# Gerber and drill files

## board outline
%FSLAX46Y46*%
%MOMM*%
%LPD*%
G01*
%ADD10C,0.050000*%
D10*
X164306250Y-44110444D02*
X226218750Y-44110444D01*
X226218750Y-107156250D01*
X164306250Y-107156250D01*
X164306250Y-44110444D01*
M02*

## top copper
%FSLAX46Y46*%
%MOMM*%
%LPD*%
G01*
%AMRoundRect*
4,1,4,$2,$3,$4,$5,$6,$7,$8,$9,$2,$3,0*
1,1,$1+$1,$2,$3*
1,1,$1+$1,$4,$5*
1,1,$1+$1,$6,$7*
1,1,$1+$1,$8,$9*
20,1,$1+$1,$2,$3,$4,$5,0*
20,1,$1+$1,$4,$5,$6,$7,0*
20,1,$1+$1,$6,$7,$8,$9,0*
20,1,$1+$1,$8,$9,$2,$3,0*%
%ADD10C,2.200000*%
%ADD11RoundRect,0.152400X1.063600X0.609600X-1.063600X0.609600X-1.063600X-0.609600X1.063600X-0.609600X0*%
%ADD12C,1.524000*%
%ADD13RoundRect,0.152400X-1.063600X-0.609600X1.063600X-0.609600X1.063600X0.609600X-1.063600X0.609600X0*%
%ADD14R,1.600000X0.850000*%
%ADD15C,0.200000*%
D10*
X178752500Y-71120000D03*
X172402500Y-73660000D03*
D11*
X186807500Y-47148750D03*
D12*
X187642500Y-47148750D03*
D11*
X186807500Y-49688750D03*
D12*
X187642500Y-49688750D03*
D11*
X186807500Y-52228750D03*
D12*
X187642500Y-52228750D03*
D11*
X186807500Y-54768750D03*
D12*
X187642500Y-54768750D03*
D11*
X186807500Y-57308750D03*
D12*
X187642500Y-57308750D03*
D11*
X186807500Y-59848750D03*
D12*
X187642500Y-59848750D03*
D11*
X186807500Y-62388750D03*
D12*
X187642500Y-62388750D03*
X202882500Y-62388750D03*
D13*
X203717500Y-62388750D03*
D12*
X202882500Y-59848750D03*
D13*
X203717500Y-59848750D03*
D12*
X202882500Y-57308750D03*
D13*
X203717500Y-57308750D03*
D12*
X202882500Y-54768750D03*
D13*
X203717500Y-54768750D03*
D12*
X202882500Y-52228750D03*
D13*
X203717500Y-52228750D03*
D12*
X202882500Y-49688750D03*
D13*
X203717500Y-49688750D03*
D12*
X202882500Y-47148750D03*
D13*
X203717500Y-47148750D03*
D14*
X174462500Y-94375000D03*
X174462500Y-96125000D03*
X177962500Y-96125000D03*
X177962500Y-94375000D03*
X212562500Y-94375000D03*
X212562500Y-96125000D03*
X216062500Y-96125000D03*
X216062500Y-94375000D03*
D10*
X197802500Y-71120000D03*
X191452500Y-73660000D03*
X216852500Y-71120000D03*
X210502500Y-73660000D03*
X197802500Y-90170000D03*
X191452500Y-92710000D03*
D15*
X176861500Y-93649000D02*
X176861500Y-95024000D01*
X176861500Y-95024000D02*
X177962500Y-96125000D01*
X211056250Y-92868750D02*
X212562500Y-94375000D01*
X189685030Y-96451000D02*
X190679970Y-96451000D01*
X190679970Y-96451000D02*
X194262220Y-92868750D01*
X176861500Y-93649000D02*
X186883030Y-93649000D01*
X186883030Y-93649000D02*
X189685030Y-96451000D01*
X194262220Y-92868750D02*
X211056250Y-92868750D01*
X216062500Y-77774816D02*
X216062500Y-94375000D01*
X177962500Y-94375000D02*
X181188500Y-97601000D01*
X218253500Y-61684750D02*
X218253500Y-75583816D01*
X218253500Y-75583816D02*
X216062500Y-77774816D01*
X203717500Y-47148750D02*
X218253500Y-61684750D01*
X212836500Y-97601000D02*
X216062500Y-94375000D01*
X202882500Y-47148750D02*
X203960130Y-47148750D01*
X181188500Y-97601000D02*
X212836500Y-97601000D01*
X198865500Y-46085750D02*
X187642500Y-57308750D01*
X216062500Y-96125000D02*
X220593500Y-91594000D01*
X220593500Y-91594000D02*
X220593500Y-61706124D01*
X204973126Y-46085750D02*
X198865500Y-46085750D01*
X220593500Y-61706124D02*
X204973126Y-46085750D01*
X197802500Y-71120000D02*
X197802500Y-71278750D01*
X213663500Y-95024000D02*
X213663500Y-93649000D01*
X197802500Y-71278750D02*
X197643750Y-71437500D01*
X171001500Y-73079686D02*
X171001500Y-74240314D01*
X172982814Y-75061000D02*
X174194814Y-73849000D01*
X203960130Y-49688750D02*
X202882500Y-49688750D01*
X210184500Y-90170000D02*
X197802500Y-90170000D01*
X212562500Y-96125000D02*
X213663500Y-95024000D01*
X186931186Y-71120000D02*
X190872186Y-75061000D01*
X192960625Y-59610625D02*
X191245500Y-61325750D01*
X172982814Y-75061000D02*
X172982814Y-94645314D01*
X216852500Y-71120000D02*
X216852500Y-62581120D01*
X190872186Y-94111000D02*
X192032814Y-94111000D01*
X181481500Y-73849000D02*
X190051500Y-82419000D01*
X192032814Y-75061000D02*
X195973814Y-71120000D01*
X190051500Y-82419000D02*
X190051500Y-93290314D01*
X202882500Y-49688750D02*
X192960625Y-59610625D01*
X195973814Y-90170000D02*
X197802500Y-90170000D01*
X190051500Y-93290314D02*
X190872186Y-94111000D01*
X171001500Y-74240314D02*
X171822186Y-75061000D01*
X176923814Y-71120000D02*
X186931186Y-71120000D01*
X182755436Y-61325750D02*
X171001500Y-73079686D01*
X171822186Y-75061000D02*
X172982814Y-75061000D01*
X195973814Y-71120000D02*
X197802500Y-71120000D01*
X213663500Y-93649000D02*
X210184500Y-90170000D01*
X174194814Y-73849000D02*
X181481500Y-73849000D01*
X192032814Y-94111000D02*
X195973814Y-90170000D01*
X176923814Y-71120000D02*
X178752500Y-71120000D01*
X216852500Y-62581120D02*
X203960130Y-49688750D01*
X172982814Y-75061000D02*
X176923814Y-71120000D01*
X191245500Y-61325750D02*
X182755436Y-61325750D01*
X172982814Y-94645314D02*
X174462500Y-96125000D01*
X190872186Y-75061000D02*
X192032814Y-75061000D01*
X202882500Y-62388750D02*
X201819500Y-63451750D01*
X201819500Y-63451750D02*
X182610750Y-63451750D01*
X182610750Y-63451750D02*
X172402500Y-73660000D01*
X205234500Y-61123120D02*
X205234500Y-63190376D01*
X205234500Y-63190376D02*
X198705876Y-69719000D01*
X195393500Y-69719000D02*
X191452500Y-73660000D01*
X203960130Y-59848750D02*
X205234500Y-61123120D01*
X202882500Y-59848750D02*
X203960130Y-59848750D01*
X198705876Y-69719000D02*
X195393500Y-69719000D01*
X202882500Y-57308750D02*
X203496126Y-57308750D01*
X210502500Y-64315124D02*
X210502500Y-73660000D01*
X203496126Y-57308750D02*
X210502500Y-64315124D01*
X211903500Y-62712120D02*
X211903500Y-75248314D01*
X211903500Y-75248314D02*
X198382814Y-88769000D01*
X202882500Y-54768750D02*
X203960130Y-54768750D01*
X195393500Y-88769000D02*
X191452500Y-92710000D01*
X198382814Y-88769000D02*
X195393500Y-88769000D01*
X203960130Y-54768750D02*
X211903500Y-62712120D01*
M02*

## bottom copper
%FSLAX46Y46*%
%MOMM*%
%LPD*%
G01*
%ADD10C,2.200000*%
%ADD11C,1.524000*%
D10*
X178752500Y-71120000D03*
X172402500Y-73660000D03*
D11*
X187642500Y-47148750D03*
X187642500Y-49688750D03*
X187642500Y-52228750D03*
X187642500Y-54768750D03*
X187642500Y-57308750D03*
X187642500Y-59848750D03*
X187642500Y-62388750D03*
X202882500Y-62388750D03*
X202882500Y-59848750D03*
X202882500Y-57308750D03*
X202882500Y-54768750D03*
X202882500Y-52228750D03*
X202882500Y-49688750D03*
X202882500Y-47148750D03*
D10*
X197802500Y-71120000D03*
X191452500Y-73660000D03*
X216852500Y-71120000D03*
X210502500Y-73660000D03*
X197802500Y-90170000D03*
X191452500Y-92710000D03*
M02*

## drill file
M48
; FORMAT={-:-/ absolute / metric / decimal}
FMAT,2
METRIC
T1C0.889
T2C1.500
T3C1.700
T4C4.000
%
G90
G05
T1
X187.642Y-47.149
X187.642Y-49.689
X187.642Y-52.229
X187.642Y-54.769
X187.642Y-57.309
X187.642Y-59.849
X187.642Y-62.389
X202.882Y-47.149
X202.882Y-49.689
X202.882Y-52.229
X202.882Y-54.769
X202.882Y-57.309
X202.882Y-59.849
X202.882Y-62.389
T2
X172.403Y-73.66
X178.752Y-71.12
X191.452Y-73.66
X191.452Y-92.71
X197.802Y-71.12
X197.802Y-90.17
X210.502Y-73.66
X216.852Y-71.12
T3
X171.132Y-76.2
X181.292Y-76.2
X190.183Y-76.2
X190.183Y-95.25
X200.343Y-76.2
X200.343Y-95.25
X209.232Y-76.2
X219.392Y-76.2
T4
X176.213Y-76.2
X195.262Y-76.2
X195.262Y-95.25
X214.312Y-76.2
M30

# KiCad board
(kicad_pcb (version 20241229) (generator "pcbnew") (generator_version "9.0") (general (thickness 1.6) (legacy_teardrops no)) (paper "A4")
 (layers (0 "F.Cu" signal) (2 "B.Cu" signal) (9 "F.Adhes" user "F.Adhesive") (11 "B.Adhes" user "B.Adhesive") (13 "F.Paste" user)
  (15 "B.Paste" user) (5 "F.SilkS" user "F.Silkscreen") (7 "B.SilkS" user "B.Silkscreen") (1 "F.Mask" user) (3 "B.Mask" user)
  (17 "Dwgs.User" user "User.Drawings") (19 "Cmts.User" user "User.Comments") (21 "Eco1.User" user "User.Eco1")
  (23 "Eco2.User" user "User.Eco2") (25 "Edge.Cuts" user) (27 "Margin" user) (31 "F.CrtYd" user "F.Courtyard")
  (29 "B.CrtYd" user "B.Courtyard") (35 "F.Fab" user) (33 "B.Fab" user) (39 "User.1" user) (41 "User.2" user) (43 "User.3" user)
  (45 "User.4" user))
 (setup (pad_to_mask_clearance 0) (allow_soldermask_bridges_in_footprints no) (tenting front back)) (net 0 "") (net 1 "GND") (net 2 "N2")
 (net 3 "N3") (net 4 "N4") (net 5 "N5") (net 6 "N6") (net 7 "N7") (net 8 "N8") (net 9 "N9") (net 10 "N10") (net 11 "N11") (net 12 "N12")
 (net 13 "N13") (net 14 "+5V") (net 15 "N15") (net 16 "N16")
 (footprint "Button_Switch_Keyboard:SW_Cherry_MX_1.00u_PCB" (layer "F.Cu") (at 178.7525 71.12)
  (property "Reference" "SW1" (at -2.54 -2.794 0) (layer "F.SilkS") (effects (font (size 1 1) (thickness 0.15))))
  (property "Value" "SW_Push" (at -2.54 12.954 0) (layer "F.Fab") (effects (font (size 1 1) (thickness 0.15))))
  (pad "" np_thru_hole circle (at -7.62 5.08) (size 1.7 1.7) (drill 1.7) (layers "*.Cu" "*.Mask"))
  (pad "" np_thru_hole circle (at -2.54 5.08) (size 4 4) (drill 4) (layers "*.Cu" "*.Mask"))
  (pad "" np_thru_hole circle (at 2.54 5.08) (size 1.7 1.7) (drill 1.7) (layers "*.Cu" "*.Mask"))
  (pad "1" thru_hole circle (at 0 0) (size 2.2 2.2) (drill 1.5) (layers "*.Cu" "*.Mask") (remove_unused_layers no) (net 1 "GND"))
  (pad "2" thru_hole circle (at -6.35 2.54) (size 2.2 2.2) (drill 1.5) (layers "*.Cu" "*.Mask") (remove_unused_layers no) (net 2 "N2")))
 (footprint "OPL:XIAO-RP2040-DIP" (layer "F.Cu") (at 195.2625 54.76875)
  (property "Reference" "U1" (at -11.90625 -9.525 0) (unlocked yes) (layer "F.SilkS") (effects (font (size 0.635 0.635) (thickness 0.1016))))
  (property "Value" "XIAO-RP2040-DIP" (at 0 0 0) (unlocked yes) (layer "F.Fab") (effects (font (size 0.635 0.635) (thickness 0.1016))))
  (pad "1" smd roundrect (at -8.455 -7.62 180) (size 2.432 1.524) (layers "F.Cu" "F.Mask") (roundrect_rratio 0.1) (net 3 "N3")
   (thermal_bridge_angle 45))
  (pad "1" thru_hole circle (at -7.62 -7.62 180) (size 1.524 1.524) (drill 0.889) (layers "*.Cu" "*.Mask") (remove_unused_layers no)
   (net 3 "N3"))
  (pad "2" smd roundrect (at -8.455 -5.08 180) (size 2.432 1.524) (layers "F.Cu" "F.Mask") (roundrect_rratio 0.1) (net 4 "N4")
   (thermal_bridge_angle 45))
  (pad "2" thru_hole circle (at -7.62 -5.08 180) (size 1.524 1.524) (drill 0.889) (layers "*.Cu" "*.Mask") (remove_unused_layers no)
   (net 4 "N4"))
  (pad "3" smd roundrect (at -8.455 -2.54 180) (size 2.432 1.524) (layers "F.Cu" "F.Mask") (roundrect_rratio 0.1) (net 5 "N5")
   (thermal_bridge_angle 45))
  (pad "3" thru_hole circle (at -7.62 -2.54 180) (size 1.524 1.524) (drill 0.889) (layers "*.Cu" "*.Mask") (remove_unused_layers no)
   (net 5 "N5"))
  (pad "4" smd roundrect (at -8.455 0 180) (size 2.432 1.524) (layers "F.Cu" "F.Mask") (roundrect_rratio 0.1) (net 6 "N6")
   (thermal_bridge_angle 45))
  (pad "4" thru_hole circle (at -7.62 0 180) (size 1.524 1.524) (drill 0.889) (layers "*.Cu" "*.Mask") (remove_unused_layers no)
   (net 6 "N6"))
  (pad "5" smd roundrect (at -8.455 2.54 180) (size 2.432 1.524) (layers "F.Cu" "F.Mask") (roundrect_rratio 0.1) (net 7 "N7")
   (thermal_bridge_angle 45))
  (pad "5" thru_hole circle (at -7.62 2.54 180) (size 1.524 1.524) (drill 0.889) (layers "*.Cu" "*.Mask") (remove_unused_layers no)
   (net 7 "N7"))
  (pad "6" smd roundrect (at -8.455 5.08 180) (size 2.432 1.524) (layers "F.Cu" "F.Mask") (roundrect_rratio 0.1) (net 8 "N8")
   (thermal_bridge_angle 45))
  (pad "6" thru_hole circle (at -7.62 5.08 180) (size 1.524 1.524) (drill 0.889) (layers "*.Cu" "*.Mask") (remove_unused_layers no)
   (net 8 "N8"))
  (pad "7" smd roundrect (at -8.455 7.62 180) (size 2.432 1.524) (layers "F.Cu" "F.Mask") (roundrect_rratio 0.1) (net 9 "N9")
   (thermal_bridge_angle 45))
  (pad "7" thru_hole circle (at -7.62 7.62 180) (size 1.524 1.524) (drill 0.889) (layers "*.Cu" "*.Mask") (remove_unused_layers no)
   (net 9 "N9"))
  (pad "8" thru_hole circle (at 7.62 7.62) (size 1.524 1.524) (drill 0.889) (layers "*.Cu" "*.Mask") (remove_unused_layers no) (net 2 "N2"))
  (pad "8" smd roundrect (at 8.455 7.62) (size 2.432 1.524) (layers "F.Cu" "F.Mask") (roundrect_rratio 0.1) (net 2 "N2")
   (thermal_bridge_angle 45))
  (pad "9" thru_hole circle (at 7.62 5.08) (size 1.524 1.524) (drill 0.889) (layers "*.Cu" "*.Mask") (remove_unused_layers no)
   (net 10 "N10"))
  (pad "9" smd roundrect (at 8.455 5.08) (size 2.432 1.524) (layers "F.Cu" "F.Mask") (roundrect_rratio 0.1) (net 10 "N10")
   (thermal_bridge_angle 45))
  (pad "10" thru_hole circle (at 7.62 2.54) (size 1.524 1.524) (drill 0.889) (layers "*.Cu" "*.Mask") (remove_unused_layers no)
   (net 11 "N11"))
  (pad "10" smd roundrect (at 8.455 2.54) (size 2.432 1.524) (layers "F.Cu" "F.Mask") (roundrect_rratio 0.1) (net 11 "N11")
   (thermal_bridge_angle 45))
  (pad "11" thru_hole circle (at 7.62 0) (size 1.524 1.524) (drill 0.889) (layers "*.Cu" "*.Mask") (remove_unused_layers no) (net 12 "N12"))
  (pad "11" smd roundrect (at 8.455 0) (size 2.432 1.524) (layers "F.Cu" "F.Mask") (roundrect_rratio 0.1) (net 12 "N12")
   (thermal_bridge_angle 45))
  (pad "12" thru_hole circle (at 7.62 -2.54) (size 1.524 1.524) (drill 0.889) (layers "*.Cu" "*.Mask") (remove_unused_layers no)
   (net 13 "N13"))
  (pad "12" smd roundrect (at 8.455 -2.54) (size 2.432 1.524) (layers "F.Cu" "F.Mask") (roundrect_rratio 0.1) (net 13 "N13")
   (thermal_bridge_angle 45))
  (pad "13" thru_hole circle (at 7.62 -5.08) (size 1.524 1.524) (drill 0.889) (layers "*.Cu" "*.Mask") (remove_unused_layers no)
   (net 1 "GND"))
  (pad "13" smd roundrect (at 8.455 -5.08) (size 2.432 1.524) (layers "F.Cu" "F.Mask") (roundrect_rratio 0.1) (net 1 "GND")
   (thermal_bridge_angle 45))
  (pad "14" thru_hole circle (at 7.62 -7.62) (size 1.524 1.524) (drill 0.889) (layers "*.Cu" "*.Mask") (remove_unused_layers no)
   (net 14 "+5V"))
  (pad "14" smd roundrect (at 8.455 -7.62) (size 2.432 1.524) (layers "F.Cu" "F.Mask") (roundrect_rratio 0.1) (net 14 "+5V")
   (thermal_bridge_angle 45)))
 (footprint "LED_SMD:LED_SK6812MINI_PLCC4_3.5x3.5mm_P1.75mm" (layer "F.Cu") (at 176.2125 95.25)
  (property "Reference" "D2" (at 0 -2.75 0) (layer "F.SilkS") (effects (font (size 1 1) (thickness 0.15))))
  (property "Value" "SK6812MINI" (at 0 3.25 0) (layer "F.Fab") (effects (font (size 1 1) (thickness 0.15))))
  (pad "1" smd rect (at -1.75 -0.875) (size 1.6 0.85) (layers "F.Cu" "F.Mask" "F.Paste") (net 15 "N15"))
  (pad "2" smd rect (at -1.75 0.875) (size 1.6 0.85) (layers "F.Cu" "F.Mask" "F.Paste") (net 1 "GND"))
  (pad "3" smd rect (at 1.75 0.875) (size 1.6 0.85) (layers "F.Cu" "F.Mask" "F.Paste") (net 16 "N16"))
  (pad "4" smd rect (at 1.75 -0.875) (size 1.6 0.85) (layers "F.Cu" "F.Mask" "F.Paste") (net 14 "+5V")))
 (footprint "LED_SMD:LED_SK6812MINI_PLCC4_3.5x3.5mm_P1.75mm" (layer "F.Cu") (at 214.3125 95.25)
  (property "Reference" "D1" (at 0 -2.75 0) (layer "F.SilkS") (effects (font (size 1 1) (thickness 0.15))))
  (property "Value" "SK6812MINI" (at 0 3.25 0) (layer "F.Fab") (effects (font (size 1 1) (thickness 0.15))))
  (pad "1" smd rect (at -1.75 -0.875) (size 1.6 0.85) (layers "F.Cu" "F.Mask" "F.Paste") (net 16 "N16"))
  (pad "2" smd rect (at -1.75 0.875) (size 1.6 0.85) (layers "F.Cu" "F.Mask" "F.Paste") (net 1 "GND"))
  (pad "3" smd rect (at 1.75 0.875) (size 1.6 0.85) (layers "F.Cu" "F.Mask" "F.Paste") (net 7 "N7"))
  (pad "4" smd rect (at 1.75 -0.875) (size 1.6 0.85) (layers "F.Cu" "F.Mask" "F.Paste") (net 14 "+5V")))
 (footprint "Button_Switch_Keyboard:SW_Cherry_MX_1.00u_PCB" (layer "F.Cu") (at 197.8025 71.12)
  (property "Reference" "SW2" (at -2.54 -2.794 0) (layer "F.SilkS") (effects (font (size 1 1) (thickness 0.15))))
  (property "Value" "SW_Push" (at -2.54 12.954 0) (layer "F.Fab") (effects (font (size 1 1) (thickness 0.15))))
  (pad "" np_thru_hole circle (at -7.62 5.08) (size 1.7 1.7) (drill 1.7) (layers "*.Cu" "*.Mask"))
  (pad "" np_thru_hole circle (at -2.54 5.08) (size 4 4) (drill 4) (layers "*.Cu" "*.Mask"))
  (pad "" np_thru_hole circle (at 2.54 5.08) (size 1.7 1.7) (drill 1.7) (layers "*.Cu" "*.Mask"))
  (pad "1" thru_hole circle (at 0 0) (size 2.2 2.2) (drill 1.5) (layers "*.Cu" "*.Mask") (remove_unused_layers no) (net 1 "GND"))
  (pad "2" thru_hole circle (at -6.35 2.54) (size 2.2 2.2) (drill 1.5) (layers "*.Cu" "*.Mask") (remove_unused_layers no) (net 10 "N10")))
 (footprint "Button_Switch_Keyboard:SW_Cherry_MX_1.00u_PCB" (layer "F.Cu") (at 216.8525 71.12)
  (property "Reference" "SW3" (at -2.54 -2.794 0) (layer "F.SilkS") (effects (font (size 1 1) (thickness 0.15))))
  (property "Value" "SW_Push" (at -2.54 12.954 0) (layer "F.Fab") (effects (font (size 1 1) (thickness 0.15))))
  (pad "" np_thru_hole circle (at -7.62 5.08) (size 1.7 1.7) (drill 1.7) (layers "*.Cu" "*.Mask"))
  (pad "" np_thru_hole circle (at -2.54 5.08) (size 4 4) (drill 4) (layers "*.Cu" "*.Mask"))
  (pad "" np_thru_hole circle (at 2.54 5.08) (size 1.7 1.7) (drill 1.7) (layers "*.Cu" "*.Mask"))
  (pad "1" thru_hole circle (at 0 0) (size 2.2 2.2) (drill 1.5) (layers "*.Cu" "*.Mask") (remove_unused_layers no) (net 1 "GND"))
  (pad "2" thru_hole circle (at -6.35 2.54) (size 2.2 2.2) (drill 1.5) (layers "*.Cu" "*.Mask") (remove_unused_layers no) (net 11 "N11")))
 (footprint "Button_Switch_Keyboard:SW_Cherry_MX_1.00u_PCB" (layer "F.Cu") (at 197.8025 90.17)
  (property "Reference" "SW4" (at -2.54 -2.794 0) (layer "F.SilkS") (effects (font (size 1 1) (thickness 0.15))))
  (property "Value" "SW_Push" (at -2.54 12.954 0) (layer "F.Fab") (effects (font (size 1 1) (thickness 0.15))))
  (pad "" np_thru_hole circle (at -7.62 5.08) (size 1.7 1.7) (drill 1.7) (layers "*.Cu" "*.Mask"))
  (pad "" np_thru_hole circle (at -2.54 5.08) (size 4 4) (drill 4) (layers "*.Cu" "*.Mask"))
  (pad "" np_thru_hole circle (at 2.54 5.08) (size 1.7 1.7) (drill 1.7) (layers "*.Cu" "*.Mask"))
  (pad "1" thru_hole circle (at 0 0) (size 2.2 2.2) (drill 1.5) (layers "*.Cu" "*.Mask") (remove_unused_layers no) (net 1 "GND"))
  (pad "2" thru_hole circle (at -6.35 2.54) (size 2.2 2.2) (drill 1.5) (layers "*.Cu" "*.Mask") (remove_unused_layers no) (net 12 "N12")))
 (gr_rect (start 164.30625 44.110444) (end 226.21875 107.15625) (stroke (width 0.05) (type default)) (fill no) (layer "Edge.Cuts"))
 (segment (start 176.8615 93.649) (end 176.8615 95.024) (width 0.2) (layer "F.Cu") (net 16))
 (segment (start 176.8615 95.024) (end 177.9625 96.125) (width 0.2) (layer "F.Cu") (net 16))
 (segment (start 211.05625 92.86875) (end 212.5625 94.375) (width 0.2) (layer "F.Cu") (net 16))
 (segment (start 189.68503 96.451) (end 190.67997 96.451) (width 0.2) (layer "F.Cu") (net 16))
 (segment (start 190.67997 96.451) (end 194.26222 92.86875) (width 0.2) (layer "F.Cu") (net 16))
 (segment (start 176.8615 93.649) (end 186.88303 93.649) (width 0.2) (layer "F.Cu") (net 16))
 (segment (start 186.88303 93.649) (end 189.68503 96.451) (width 0.2) (layer "F.Cu") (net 16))
 (segment (start 194.26222 92.86875) (end 211.05625 92.86875) (width 0.2) (layer "F.Cu") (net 16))
 (segment (start 216.0625 77.774816) (end 216.0625 94.375) (width 0.2) (layer "F.Cu") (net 14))
 (segment (start 177.9625 94.375) (end 181.1885 97.601) (width 0.2) (layer "F.Cu") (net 14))
 (segment (start 218.2535 61.68475) (end 218.2535 75.583816) (width 0.2) (layer "F.Cu") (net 14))
 (segment (start 218.2535 75.583816) (end 216.0625 77.774816) (width 0.2) (layer "F.Cu") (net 14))
 (segment (start 203.7175 47.14875) (end 218.2535 61.68475) (width 0.2) (layer "F.Cu") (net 14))
 (segment (start 212.8365 97.601) (end 216.0625 94.375) (width 0.2) (layer "F.Cu") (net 14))
 (segment (start 202.8825 47.14875) (end 203.96013 47.14875) (width 0.2) (layer "F.Cu") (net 14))
 (segment (start 181.1885 97.601) (end 212.8365 97.601) (width 0.2) (layer "F.Cu") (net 14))
 (segment (start 198.8655 46.08575) (end 187.6425 57.30875) (width 0.2) (layer "F.Cu") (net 7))
 (segment (start 216.0625 96.125) (end 220.5935 91.594) (width 0.2) (layer "F.Cu") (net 7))
 (segment (start 220.5935 91.594) (end 220.5935 61.706124) (width 0.2) (layer "F.Cu") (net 7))
 (segment (start 204.973126 46.08575) (end 198.8655 46.08575) (width 0.2) (layer "F.Cu") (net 7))
 (segment (start 220.5935 61.706124) (end 204.973126 46.08575) (width 0.2) (layer "F.Cu") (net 7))
 (segment (start 197.8025 71.12) (end 197.8025 71.27875) (width 0.2) (layer "F.Cu") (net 1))
 (segment (start 213.6635 95.024) (end 213.6635 93.649) (width 0.2) (layer "F.Cu") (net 1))
 (segment (start 197.8025 71.27875) (end 197.64375 71.4375) (width 0.2) (layer "F.Cu") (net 1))
 (segment (start 171.0015 73.079686) (end 171.0015 74.240314) (width 0.2) (layer "F.Cu") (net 1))
 (segment (start 172.982814 75.061) (end 174.194814 73.849) (width 0.2) (layer "F.Cu") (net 1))
 (segment (start 203.96013 49.68875) (end 202.8825 49.68875) (width 0.2) (layer "F.Cu") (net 1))
 (segment (start 210.1845 90.17) (end 197.8025 90.17) (width 0.2) (layer "F.Cu") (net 1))
 (segment (start 212.5625 96.125) (end 213.6635 95.024) (width 0.2) (layer "F.Cu") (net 1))
 (segment (start 186.931186 71.12) (end 190.872186 75.061) (width 0.2) (layer "F.Cu") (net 1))
 (segment (start 192.960625 59.610625) (end 191.2455 61.32575) (width 0.2) (layer "F.Cu") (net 1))
 (segment (start 172.982814 75.061) (end 172.982814 94.645314) (width 0.2) (layer "F.Cu") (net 1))
 (segment (start 216.8525 71.12) (end 216.8525 62.58112) (width 0.2) (layer "F.Cu") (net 1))
 (segment (start 190.872186 94.111) (end 192.032814 94.111) (width 0.2) (layer "F.Cu") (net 1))
 (segment (start 181.4815 73.849) (end 190.0515 82.419) (width 0.2) (layer "F.Cu") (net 1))
 (segment (start 192.032814 75.061) (end 195.973814 71.12) (width 0.2) (layer "F.Cu") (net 1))
 (segment (start 190.0515 82.419) (end 190.0515 93.290314) (width 0.2) (layer "F.Cu") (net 1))
 (segment (start 202.8825 49.68875) (end 192.960625 59.610625) (width 0.2) (layer "F.Cu") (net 1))
 (segment (start 195.973814 90.17) (end 197.8025 90.17) (width 0.2) (layer "F.Cu") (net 1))
 (segment (start 190.0515 93.290314) (end 190.872186 94.111) (width 0.2) (layer "F.Cu") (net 1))
 (segment (start 171.0015 74.240314) (end 171.822186 75.061) (width 0.2) (layer "F.Cu") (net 1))
 (segment (start 176.923814 71.12) (end 186.931186 71.12) (width 0.2) (layer "F.Cu") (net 1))
 (segment (start 182.755436 61.32575) (end 171.0015 73.079686) (width 0.2) (layer "F.Cu") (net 1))
 (segment (start 171.822186 75.061) (end 172.982814 75.061) (width 0.2) (layer "F.Cu") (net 1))
 (segment (start 195.973814 71.12) (end 197.8025 71.12) (width 0.2) (layer "F.Cu") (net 1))
 (segment (start 213.6635 93.649) (end 210.1845 90.17) (width 0.2) (layer "F.Cu") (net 1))
 (segment (start 174.194814 73.849) (end 181.4815 73.849) (width 0.2) (layer "F.Cu") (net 1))
 (segment (start 192.032814 94.111) (end 195.973814 90.17) (width 0.2) (layer "F.Cu") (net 1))
 (segment (start 176.923814 71.12) (end 178.7525 71.12) (width 0.2) (layer "F.Cu") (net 1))
 (segment (start 216.8525 62.58112) (end 203.96013 49.68875) (width 0.2) (layer "F.Cu") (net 1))
 (segment (start 172.982814 75.061) (end 176.923814 71.12) (width 0.2) (layer "F.Cu") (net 1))
 (segment (start 191.2455 61.32575) (end 182.755436 61.32575) (width 0.2) (layer "F.Cu") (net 1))
 (segment (start 172.982814 94.645314) (end 174.4625 96.125) (width 0.2) (layer "F.Cu") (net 1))
 (segment (start 190.872186 75.061) (end 192.032814 75.061) (width 0.2) (layer "F.Cu") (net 1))
 (segment (start 202.8825 62.38875) (end 201.8195 63.45175) (width 0.2) (layer "F.Cu") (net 2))
 (segment (start 201.8195 63.45175) (end 182.61075 63.45175) (width 0.2) (layer "F.Cu") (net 2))
 (segment (start 182.61075 63.45175) (end 172.4025 73.66) (width 0.2) (layer "F.Cu") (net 2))
 (segment (start 205.2345 61.12312) (end 205.2345 63.190376) (width 0.2) (layer "F.Cu") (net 10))
 (segment (start 205.2345 63.190376) (end 198.705876 69.719) (width 0.2) (layer "F.Cu") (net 10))
 (segment (start 195.3935 69.719) (end 191.4525 73.66) (width 0.2) (layer "F.Cu") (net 10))
 (segment (start 203.96013 59.84875) (end 205.2345 61.12312) (width 0.2) (layer "F.Cu") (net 10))
 (segment (start 202.8825 59.84875) (end 203.96013 59.84875) (width 0.2) (layer "F.Cu") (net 10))
 (segment (start 198.705876 69.719) (end 195.3935 69.719) (width 0.2) (layer "F.Cu") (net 10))
 (segment (start 202.8825 57.30875) (end 203.496126 57.30875) (width 0.2) (layer "F.Cu") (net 11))
 (segment (start 210.5025 64.315124) (end 210.5025 73.66) (width 0.2) (layer "F.Cu") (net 11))
 (segment (start 203.496126 57.30875) (end 210.5025 64.315124) (width 0.2) (layer "F.Cu") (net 11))
 (segment (start 211.9035 62.71212) (end 211.9035 75.248314) (width 0.2) (layer "F.Cu") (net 12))
 (segment (start 211.9035 75.248314) (end 198.382814 88.769) (width 0.2) (layer "F.Cu") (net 12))
 (segment (start 202.8825 54.76875) (end 203.96013 54.76875) (width 0.2) (layer "F.Cu") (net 12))
 (segment (start 195.3935 88.769) (end 191.4525 92.71) (width 0.2) (layer "F.Cu") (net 12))
 (segment (start 198.382814 88.769) (end 195.3935 88.769) (width 0.2) (layer "F.Cu") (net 12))
 (segment (start 203.96013 54.76875) (end 211.9035 62.71212) (width 0.2) (layer "F.Cu") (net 12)))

